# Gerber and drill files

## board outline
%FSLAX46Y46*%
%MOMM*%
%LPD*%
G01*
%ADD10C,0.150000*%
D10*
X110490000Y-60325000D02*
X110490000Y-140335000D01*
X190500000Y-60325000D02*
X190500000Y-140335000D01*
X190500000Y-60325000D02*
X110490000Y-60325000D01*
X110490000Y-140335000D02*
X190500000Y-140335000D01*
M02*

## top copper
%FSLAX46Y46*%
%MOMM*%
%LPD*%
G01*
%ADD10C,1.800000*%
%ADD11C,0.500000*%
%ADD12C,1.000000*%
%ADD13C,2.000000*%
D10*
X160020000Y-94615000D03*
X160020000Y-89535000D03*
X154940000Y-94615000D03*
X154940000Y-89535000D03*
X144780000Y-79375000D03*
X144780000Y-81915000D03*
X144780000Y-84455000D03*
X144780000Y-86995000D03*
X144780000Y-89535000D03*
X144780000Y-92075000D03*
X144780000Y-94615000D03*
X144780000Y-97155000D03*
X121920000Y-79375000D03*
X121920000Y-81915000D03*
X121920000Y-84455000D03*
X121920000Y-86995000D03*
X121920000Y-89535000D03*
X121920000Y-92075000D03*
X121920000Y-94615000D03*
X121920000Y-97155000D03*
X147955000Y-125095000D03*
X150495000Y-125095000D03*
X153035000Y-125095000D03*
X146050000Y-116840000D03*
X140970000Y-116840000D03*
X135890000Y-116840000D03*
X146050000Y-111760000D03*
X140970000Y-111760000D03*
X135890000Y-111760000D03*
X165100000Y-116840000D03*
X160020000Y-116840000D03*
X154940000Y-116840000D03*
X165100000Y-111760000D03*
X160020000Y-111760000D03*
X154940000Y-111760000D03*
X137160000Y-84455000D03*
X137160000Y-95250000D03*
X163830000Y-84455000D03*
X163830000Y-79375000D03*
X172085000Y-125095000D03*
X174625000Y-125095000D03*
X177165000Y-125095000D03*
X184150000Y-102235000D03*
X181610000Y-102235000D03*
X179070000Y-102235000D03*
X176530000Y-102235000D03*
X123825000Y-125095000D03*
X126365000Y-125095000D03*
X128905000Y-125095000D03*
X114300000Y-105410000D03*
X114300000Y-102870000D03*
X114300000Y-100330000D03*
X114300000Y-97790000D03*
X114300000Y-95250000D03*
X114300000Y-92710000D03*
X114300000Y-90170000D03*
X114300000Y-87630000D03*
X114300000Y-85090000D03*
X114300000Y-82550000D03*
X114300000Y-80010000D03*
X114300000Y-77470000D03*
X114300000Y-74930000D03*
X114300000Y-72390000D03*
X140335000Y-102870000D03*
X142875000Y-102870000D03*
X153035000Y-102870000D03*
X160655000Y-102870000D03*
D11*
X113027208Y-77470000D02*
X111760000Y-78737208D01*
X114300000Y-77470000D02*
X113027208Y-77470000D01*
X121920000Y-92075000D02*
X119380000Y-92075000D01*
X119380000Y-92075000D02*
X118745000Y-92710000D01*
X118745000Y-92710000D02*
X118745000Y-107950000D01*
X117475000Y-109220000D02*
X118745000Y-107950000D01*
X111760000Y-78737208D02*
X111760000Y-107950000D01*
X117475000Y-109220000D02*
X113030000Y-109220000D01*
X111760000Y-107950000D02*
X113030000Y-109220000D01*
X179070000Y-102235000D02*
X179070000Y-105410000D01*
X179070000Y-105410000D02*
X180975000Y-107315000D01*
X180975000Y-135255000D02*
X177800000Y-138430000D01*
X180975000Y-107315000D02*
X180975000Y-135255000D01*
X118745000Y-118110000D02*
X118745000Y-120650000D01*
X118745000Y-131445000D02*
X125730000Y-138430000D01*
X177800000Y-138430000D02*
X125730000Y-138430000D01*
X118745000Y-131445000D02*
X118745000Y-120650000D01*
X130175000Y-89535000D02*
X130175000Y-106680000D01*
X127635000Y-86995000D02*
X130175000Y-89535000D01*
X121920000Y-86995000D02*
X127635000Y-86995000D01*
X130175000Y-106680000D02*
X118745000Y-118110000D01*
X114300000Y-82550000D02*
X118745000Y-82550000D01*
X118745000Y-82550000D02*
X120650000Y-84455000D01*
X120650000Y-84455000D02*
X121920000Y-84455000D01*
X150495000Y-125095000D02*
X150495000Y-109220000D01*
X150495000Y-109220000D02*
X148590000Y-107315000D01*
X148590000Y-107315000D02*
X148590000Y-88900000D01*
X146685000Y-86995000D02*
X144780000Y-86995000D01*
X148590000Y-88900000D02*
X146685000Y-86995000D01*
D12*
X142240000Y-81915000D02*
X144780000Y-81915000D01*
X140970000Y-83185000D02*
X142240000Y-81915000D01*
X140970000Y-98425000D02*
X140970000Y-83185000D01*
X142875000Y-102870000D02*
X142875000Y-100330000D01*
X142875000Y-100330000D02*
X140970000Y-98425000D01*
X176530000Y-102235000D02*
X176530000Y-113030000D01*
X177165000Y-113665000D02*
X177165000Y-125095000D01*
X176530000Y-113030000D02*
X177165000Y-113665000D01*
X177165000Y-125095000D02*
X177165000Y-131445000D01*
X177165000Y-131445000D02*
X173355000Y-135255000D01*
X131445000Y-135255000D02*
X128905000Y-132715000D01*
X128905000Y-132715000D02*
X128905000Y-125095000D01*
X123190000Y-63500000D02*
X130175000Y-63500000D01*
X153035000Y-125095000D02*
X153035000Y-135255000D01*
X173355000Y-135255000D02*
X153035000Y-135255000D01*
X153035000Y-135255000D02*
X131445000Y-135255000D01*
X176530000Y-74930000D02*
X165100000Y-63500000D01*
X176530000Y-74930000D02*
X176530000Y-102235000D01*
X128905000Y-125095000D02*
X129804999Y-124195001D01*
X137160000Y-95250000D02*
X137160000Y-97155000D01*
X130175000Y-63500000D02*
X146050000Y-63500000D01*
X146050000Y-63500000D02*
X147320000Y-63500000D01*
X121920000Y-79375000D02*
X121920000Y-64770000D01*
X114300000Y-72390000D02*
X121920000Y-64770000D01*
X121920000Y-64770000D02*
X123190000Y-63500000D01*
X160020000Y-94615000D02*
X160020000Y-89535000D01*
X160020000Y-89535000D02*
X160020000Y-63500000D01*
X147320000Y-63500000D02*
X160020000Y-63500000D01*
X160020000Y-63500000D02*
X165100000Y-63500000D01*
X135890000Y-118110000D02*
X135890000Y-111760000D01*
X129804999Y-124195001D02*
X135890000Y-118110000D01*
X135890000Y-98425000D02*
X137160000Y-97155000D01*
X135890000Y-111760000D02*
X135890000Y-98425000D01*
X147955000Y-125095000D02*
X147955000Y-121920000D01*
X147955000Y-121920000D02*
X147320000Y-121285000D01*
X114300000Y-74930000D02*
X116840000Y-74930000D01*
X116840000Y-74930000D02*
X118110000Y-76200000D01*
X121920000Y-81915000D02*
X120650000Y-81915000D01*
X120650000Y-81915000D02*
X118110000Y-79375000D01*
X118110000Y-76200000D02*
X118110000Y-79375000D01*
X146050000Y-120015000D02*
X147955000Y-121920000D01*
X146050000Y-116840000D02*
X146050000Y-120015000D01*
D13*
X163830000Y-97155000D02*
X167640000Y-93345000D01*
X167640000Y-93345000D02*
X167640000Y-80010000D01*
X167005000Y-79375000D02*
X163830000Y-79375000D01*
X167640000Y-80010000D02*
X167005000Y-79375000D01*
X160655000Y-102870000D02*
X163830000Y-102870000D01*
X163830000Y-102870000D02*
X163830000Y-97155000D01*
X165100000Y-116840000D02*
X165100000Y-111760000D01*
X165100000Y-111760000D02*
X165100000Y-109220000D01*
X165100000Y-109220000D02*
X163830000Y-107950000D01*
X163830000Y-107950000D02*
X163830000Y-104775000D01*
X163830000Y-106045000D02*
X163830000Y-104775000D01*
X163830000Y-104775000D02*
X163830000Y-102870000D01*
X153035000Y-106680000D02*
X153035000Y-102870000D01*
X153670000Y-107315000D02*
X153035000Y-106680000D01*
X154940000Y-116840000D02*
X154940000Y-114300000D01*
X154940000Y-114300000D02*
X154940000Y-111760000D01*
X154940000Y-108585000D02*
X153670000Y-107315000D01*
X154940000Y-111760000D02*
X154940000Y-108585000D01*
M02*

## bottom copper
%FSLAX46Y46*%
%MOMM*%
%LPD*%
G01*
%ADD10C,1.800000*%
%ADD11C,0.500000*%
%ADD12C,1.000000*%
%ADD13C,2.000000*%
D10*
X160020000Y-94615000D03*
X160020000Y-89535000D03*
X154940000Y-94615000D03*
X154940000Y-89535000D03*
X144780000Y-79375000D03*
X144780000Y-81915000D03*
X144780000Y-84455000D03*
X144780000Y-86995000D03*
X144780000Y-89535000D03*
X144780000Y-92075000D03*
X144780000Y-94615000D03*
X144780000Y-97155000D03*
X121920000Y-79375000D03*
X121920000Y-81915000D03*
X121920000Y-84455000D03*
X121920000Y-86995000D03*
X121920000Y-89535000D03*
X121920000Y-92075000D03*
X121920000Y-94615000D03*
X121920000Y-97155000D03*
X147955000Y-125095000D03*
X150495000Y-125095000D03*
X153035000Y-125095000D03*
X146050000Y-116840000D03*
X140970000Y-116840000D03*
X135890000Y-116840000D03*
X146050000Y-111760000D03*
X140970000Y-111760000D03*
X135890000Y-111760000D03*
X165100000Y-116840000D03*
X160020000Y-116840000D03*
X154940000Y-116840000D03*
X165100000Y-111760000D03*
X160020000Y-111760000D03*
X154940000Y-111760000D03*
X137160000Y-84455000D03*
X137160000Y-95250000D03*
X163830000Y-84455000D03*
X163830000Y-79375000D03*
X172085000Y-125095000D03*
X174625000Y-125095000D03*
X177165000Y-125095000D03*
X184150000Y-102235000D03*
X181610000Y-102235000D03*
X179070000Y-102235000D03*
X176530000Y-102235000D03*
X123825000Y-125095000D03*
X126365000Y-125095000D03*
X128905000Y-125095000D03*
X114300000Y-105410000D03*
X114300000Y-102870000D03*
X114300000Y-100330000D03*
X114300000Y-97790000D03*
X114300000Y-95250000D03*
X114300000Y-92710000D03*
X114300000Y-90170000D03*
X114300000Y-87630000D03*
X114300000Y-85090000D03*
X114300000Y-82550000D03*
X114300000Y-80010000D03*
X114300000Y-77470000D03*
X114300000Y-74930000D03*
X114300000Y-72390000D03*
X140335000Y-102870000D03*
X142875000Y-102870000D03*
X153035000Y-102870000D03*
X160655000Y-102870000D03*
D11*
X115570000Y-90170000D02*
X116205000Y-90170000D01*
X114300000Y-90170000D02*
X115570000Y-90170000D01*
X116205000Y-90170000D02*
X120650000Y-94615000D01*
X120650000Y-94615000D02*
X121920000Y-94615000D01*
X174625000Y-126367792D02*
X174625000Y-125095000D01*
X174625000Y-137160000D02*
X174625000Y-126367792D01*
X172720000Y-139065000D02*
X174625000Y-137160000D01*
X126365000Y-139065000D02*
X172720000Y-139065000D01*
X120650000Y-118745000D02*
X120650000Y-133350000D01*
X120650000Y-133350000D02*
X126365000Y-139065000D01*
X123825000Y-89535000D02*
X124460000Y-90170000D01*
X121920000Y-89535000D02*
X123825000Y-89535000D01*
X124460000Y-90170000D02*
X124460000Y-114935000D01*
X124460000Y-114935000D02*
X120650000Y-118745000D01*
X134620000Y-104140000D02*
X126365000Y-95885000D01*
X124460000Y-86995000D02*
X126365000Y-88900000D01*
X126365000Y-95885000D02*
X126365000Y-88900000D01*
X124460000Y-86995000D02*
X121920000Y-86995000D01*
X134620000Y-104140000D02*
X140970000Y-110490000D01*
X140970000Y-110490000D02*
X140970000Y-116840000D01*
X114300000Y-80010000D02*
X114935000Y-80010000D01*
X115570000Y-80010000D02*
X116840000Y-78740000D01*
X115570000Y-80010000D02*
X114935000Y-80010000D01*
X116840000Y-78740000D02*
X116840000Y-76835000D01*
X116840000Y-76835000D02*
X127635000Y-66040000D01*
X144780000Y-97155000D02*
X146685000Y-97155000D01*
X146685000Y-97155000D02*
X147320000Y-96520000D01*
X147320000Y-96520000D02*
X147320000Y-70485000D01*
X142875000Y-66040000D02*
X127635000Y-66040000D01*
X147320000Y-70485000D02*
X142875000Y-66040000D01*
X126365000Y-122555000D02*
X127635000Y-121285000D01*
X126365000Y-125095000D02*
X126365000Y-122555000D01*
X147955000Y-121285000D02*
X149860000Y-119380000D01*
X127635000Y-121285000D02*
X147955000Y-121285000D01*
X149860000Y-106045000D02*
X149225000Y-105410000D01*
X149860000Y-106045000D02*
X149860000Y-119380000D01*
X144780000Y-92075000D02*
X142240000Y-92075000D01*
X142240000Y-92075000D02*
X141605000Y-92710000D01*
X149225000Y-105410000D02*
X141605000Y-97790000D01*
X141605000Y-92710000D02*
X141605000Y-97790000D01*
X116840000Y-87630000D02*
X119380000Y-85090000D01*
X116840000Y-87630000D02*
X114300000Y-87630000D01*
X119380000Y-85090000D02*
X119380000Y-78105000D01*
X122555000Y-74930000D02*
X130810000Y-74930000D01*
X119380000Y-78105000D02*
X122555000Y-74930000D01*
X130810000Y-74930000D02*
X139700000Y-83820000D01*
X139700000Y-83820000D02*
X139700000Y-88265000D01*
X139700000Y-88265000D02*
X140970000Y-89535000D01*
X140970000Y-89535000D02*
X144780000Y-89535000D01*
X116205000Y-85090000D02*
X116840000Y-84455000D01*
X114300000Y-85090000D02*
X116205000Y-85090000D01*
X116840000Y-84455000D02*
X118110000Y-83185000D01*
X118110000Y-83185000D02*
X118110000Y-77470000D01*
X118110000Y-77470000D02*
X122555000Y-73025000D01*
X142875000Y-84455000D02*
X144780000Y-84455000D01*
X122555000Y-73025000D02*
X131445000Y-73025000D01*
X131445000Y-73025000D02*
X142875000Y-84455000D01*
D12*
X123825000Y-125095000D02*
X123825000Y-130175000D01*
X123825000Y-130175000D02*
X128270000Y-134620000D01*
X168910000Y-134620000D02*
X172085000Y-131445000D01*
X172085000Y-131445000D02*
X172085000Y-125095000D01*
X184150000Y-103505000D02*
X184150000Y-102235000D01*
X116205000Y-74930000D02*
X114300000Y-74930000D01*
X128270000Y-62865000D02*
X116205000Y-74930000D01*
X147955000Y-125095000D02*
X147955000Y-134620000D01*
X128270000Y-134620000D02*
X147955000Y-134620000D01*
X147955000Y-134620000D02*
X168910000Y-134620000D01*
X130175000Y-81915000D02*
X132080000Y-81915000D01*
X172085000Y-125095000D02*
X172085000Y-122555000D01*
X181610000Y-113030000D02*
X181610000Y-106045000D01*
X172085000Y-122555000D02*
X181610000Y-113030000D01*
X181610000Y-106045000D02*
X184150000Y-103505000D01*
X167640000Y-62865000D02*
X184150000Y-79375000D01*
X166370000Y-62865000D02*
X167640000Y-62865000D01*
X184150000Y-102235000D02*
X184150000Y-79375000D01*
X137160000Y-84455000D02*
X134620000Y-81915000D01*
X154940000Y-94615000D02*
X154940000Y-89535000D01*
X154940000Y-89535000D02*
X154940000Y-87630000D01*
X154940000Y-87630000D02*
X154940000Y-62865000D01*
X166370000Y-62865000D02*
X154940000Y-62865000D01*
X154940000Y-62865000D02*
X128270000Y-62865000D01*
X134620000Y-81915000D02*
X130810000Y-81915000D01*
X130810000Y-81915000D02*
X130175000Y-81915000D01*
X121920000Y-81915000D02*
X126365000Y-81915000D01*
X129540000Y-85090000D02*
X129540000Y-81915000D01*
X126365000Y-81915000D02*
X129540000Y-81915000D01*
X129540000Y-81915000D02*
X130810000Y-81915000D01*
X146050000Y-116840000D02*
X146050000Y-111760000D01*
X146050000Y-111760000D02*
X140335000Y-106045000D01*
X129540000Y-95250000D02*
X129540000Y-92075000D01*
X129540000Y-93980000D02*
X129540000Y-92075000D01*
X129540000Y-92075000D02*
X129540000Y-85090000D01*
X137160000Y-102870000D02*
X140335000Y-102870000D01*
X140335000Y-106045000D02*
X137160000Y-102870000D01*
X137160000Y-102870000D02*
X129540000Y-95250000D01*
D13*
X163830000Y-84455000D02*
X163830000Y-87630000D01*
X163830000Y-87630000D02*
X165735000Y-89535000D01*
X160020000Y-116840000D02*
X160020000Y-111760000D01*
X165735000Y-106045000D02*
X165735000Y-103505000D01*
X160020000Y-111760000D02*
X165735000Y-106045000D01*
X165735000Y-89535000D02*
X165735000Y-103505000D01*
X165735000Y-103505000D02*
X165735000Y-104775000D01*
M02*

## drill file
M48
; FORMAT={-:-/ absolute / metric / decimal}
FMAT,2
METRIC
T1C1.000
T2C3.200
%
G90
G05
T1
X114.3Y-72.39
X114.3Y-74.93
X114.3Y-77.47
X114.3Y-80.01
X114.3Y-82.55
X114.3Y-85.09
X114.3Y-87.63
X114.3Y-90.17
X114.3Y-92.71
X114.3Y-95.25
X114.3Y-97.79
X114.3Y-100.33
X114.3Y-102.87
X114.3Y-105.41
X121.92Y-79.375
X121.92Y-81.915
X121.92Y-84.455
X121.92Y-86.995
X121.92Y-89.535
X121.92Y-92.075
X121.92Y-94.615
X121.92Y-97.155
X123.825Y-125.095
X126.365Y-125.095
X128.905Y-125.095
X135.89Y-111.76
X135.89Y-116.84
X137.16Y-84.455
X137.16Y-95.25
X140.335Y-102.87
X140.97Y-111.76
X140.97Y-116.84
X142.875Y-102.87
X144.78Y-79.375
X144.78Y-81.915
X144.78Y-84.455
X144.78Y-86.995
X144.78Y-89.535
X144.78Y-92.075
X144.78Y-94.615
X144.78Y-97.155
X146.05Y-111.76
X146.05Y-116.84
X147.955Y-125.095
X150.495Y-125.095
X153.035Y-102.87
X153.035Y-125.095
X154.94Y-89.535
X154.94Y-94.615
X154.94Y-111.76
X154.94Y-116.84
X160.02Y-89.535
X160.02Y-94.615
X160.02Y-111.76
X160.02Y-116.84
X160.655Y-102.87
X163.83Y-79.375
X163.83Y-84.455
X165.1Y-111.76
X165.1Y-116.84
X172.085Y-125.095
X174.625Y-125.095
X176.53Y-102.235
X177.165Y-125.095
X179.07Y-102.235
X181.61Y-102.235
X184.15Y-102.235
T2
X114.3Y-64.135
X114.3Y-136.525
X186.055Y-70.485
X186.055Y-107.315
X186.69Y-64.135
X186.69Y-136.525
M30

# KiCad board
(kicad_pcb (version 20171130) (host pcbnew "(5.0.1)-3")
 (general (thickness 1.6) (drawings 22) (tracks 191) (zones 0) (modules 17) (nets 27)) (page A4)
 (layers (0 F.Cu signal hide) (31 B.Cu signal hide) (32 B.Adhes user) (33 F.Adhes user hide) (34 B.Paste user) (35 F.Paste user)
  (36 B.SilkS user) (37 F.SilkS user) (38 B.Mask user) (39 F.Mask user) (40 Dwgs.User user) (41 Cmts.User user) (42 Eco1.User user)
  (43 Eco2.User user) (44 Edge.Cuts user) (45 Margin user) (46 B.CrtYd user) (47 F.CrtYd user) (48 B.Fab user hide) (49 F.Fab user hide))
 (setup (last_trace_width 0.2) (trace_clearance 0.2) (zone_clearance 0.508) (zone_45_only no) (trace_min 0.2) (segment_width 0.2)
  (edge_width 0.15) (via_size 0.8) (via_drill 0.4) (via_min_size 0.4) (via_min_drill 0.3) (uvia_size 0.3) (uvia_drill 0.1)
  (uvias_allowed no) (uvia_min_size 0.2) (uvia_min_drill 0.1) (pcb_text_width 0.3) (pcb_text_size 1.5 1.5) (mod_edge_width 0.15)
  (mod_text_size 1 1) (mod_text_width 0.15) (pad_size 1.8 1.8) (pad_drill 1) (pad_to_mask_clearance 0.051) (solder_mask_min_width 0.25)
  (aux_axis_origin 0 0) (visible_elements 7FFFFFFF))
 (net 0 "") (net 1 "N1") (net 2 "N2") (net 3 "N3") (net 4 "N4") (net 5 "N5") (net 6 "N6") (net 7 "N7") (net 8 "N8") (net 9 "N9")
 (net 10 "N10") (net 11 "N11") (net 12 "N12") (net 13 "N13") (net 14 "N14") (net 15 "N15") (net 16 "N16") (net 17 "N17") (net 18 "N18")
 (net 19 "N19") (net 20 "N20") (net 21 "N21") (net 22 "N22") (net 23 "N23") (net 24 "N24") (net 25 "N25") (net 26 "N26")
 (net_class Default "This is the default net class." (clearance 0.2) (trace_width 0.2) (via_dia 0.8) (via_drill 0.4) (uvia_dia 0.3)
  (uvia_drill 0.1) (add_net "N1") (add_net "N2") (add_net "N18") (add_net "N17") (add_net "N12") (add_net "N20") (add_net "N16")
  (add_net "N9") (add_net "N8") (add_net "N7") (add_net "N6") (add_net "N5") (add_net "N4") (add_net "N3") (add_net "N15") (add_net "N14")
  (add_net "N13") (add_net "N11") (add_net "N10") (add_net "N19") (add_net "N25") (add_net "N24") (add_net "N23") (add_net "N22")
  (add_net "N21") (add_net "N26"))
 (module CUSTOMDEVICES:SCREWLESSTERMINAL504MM (layer B.Cu) (at 154.94 92.075 180)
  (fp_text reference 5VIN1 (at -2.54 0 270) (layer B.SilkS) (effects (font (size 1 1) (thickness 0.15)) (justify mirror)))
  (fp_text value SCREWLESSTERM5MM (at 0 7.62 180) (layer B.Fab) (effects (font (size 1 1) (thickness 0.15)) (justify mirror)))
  (pad 1 thru_hole circle (at -5.08 -2.54 180) (size 1.8 1.8) (drill 1) (layers *.Cu *.Mask) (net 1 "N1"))
  (pad 1 thru_hole circle (at -5.08 2.54 180) (size 1.8 1.8) (drill 1) (layers *.Cu *.Mask) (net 1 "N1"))
  (pad 2 thru_hole circle (at 0 -2.54 180) (size 1.8 1.8) (drill 1) (layers *.Cu *.Mask) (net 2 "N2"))
  (pad 2 thru_hole circle (at 0 2.54 180) (size 1.8 1.8) (drill 1) (layers *.Cu *.Mask) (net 2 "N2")))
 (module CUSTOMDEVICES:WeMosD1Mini (layer F.Cu) (at 133.35 86.995 180)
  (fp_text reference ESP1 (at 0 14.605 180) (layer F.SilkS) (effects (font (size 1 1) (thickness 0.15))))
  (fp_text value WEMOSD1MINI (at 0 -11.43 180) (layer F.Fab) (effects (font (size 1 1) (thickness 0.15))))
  (pad 16 thru_hole circle (at -11.43 7.62 180) (size 1.8 1.8) (drill 1) (layers *.Cu *.Mask) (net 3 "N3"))
  (pad 15 thru_hole circle (at -11.43 5.08 180) (size 1.8 1.8) (drill 1) (layers *.Cu *.Mask) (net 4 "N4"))
  (pad 14 thru_hole circle (at -11.43 2.54 180) (size 1.8 1.8) (drill 1) (layers *.Cu *.Mask) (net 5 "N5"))
  (pad 13 thru_hole circle (at -11.43 0 180) (size 1.8 1.8) (drill 1) (layers *.Cu *.Mask) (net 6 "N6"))
  (pad 12 thru_hole circle (at -11.43 -2.54 180) (size 1.8 1.8) (drill 1) (layers *.Cu *.Mask) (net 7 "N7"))
  (pad 11 thru_hole circle (at -11.43 -5.08 180) (size 1.8 1.8) (drill 1) (layers *.Cu *.Mask) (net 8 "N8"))
  (pad 10 thru_hole circle (at -11.43 -7.62 180) (size 1.8 1.8) (drill 1) (layers *.Cu *.Mask) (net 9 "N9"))
  (pad 9 thru_hole circle (at -11.43 -10.16 180) (size 1.8 1.8) (drill 1) (layers *.Cu *.Mask) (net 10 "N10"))
  (pad 8 thru_hole circle (at 11.43 7.62 180) (size 1.8 1.8) (drill 1) (layers *.Cu *.Mask) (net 1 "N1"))
  (pad 7 thru_hole circle (at 11.43 5.08 180) (size 1.8 1.8) (drill 1) (layers *.Cu *.Mask) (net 2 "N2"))
  (pad 6 thru_hole circle (at 11.43 2.54 180) (size 1.8 1.8) (drill 1) (layers *.Cu *.Mask) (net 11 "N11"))
  (pad 5 thru_hole circle (at 11.43 0 180) (size 1.8 1.8) (drill 1) (layers *.Cu *.Mask) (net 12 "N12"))
  (pad 4 thru_hole circle (at 11.43 -2.54 180) (size 1.8 1.8) (drill 1) (layers *.Cu *.Mask) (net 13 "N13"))
  (pad 3 thru_hole circle (at 11.43 -5.08 180) (size 1.8 1.8) (drill 1) (layers *.Cu *.Mask) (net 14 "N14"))
  (pad 2 thru_hole circle (at 11.43 -7.62 180) (size 1.8 1.8) (drill 1) (layers *.Cu *.Mask) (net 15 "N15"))
  (pad 1 thru_hole circle (at 11.43 -10.16 180) (size 1.8 1.8) (drill 1) (layers *.Cu *.Mask) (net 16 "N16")))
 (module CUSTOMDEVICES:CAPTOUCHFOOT (layer F.Cu) (at 150.495 130.175 180)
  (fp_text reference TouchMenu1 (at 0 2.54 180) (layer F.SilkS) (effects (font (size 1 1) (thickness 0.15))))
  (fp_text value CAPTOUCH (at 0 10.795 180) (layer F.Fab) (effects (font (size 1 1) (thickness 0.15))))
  (pad 3 thru_hole circle (at 2.54 5.08 180) (size 1.8 1.8) (drill 1) (layers *.Cu *.Mask) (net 2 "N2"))
  (pad 2 thru_hole circle (at 0 5.08 180) (size 1.8 1.8) (drill 1) (layers *.Cu *.Mask) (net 6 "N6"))
  (pad 1 thru_hole circle (at -2.54 5.08 180) (size 1.8 1.8) (drill 1) (layers *.Cu *.Mask) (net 1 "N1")))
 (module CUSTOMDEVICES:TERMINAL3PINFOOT (layer B.Cu) (at 140.97 114.3)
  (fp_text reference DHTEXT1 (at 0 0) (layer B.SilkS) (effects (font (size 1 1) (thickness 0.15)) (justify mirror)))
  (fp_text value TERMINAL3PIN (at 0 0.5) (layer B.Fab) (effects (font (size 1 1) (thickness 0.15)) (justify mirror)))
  (pad 3 thru_hole circle (at 5.08 2.54) (size 1.8 1.8) (drill 1) (layers *.Cu *.Mask) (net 2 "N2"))
  (pad 2 thru_hole circle (at 0 2.54) (size 1.8 1.8) (drill 1) (layers *.Cu *.Mask) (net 12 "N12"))
  (pad 1 thru_hole circle (at -5.08 2.54) (size 1.8 1.8) (drill 1) (layers *.Cu *.Mask) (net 1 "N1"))
  (pad 3 thru_hole circle (at 5.08 -2.54) (size 1.8 1.8) (drill 1) (layers *.Cu *.Mask) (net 2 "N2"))
  (pad 2 thru_hole circle (at 0 -2.54) (size 1.8 1.8) (drill 1) (layers *.Cu *.Mask) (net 12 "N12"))
  (pad 1 thru_hole circle (at -5.08 -2.54) (size 1.8 1.8) (drill 1) (layers *.Cu *.Mask) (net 1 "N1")))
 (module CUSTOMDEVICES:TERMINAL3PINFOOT (layer B.Cu) (at 160.02 114.3)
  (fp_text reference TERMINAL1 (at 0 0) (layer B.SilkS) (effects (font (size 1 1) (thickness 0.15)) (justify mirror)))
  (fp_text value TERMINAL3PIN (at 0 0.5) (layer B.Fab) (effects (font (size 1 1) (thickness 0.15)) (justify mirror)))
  (pad 3 thru_hole circle (at 5.08 2.54) (size 1.8 1.8) (drill 1) (layers *.Cu *.Mask) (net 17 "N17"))
  (pad 2 thru_hole circle (at 0 2.54) (size 1.8 1.8) (drill 1) (layers *.Cu *.Mask) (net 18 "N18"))
  (pad 1 thru_hole circle (at -5.08 2.54) (size 1.8 1.8) (drill 1) (layers *.Cu *.Mask) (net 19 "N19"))
  (pad 3 thru_hole circle (at 5.08 -2.54) (size 1.8 1.8) (drill 1) (layers *.Cu *.Mask) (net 17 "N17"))
  (pad 2 thru_hole circle (at 0 -2.54) (size 1.8 1.8) (drill 1) (layers *.Cu *.Mask) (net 18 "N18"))
  (pad 1 thru_hole circle (at -5.08 -2.54) (size 1.8 1.8) (drill 1) (layers *.Cu *.Mask) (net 19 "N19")))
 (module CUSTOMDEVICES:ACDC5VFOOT (layer B.Cu) (at 157.48 86.995 90)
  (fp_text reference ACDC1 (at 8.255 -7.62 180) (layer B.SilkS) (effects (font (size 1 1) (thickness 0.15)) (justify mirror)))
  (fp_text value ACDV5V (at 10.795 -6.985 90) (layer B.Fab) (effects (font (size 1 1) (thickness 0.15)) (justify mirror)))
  (pad 3 thru_hole circle (at 2.54 -20.32 90) (size 1.8 1.8) (drill 1) (layers *.Cu *.Mask) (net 2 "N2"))
  (pad 4 thru_hole circle (at -8.255 -20.32 90) (size 1.8 1.8) (drill 1) (layers *.Cu *.Mask) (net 1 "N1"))
  (pad 1 thru_hole circle (at 2.54 6.35 90) (size 1.8 1.8) (drill 1) (layers *.Cu *.Mask) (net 18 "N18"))
  (pad 2 thru_hole circle (at 7.62 6.35 90) (size 1.8 1.8) (drill 1) (layers *.Cu *.Mask) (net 17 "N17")))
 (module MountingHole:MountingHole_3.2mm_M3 (layer F.Cu) (at 186.055 107.315)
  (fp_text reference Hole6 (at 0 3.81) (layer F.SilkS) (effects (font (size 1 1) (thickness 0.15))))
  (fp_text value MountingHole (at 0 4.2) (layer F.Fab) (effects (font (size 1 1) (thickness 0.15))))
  (pad 1 np_thru_hole circle (at 0 0) (size 3.2 3.2) (drill 3.2) (layers *.Cu *.Mask)))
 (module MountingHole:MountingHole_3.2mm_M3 (layer F.Cu) (at 186.055 70.485)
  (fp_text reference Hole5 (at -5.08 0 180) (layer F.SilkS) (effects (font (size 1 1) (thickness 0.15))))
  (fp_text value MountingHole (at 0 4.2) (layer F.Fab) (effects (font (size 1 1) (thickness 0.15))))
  (pad 1 np_thru_hole circle (at 0 0) (size 3.2 3.2) (drill 3.2) (layers *.Cu *.Mask)))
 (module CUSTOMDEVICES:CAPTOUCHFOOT (layer F.Cu) (at 174.625 130.175 180)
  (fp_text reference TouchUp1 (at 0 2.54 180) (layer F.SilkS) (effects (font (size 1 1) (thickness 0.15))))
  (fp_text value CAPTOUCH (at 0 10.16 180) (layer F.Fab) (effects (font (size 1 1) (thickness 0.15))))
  (pad 3 thru_hole circle (at 2.54 5.08 180) (size 1.8 1.8) (drill 1) (layers *.Cu *.Mask) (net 2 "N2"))
  (pad 2 thru_hole circle (at 0 5.08 180) (size 1.8 1.8) (drill 1) (layers *.Cu *.Mask) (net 13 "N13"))
  (pad 1 thru_hole circle (at -2.54 5.08 180) (size 1.8 1.8) (drill 1) (layers *.Cu *.Mask) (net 1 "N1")))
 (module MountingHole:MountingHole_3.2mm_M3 (layer F.Cu) (at 186.69 136.525)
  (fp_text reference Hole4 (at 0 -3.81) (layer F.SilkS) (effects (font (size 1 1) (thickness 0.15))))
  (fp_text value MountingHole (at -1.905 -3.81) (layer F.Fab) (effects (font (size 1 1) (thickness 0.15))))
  (pad 1 np_thru_hole circle (at 0 0) (size 3.2 3.2) (drill 3.2) (layers *.Cu *.Mask)))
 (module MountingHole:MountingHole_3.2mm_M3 (layer F.Cu) (at 114.3 136.525)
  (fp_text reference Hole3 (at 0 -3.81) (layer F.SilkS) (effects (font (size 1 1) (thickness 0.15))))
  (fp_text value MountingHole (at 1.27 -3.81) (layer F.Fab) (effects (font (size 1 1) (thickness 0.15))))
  (pad 1 np_thru_hole circle (at 0 0) (size 3.2 3.2) (drill 3.2) (layers *.Cu *.Mask)))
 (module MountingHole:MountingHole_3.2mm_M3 (layer F.Cu) (at 186.69 64.135)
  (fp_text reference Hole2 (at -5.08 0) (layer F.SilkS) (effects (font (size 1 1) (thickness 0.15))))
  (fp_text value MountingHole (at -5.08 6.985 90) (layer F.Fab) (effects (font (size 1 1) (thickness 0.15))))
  (pad 1 np_thru_hole circle (at 0 0) (size 3.2 3.2) (drill 3.2) (layers *.Cu *.Mask)))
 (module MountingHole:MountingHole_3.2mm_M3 (layer F.Cu) (at 114.3 64.135)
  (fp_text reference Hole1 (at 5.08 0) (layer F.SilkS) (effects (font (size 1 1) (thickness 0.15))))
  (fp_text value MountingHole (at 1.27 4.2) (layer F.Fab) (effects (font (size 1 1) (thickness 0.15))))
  (pad 1 np_thru_hole circle (at 0 0) (size 3.2 3.2) (drill 3.2) (layers *.Cu *.Mask)))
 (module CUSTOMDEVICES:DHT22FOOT (layer F.Cu) (at 181.61 89.535)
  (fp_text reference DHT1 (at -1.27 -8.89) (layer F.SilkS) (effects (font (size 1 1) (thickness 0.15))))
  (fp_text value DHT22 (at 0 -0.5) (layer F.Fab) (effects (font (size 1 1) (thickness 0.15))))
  (pad 4 thru_hole circle (at 2.54 12.7) (size 1.8 1.8) (drill 1) (layers *.Cu *.Mask) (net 2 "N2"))
  (pad 3 thru_hole circle (at 0 12.7) (size 1.8 1.8) (drill 1) (layers *.Cu *.Mask) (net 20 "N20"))
  (pad 2 thru_hole circle (at -2.54 12.7) (size 1.8 1.8) (drill 1) (layers *.Cu *.Mask) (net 12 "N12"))
  (pad 1 thru_hole circle (at -5.08 12.7) (size 1.8 1.8) (drill 1) (layers *.Cu *.Mask) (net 1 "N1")))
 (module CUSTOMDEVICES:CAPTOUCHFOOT (layer F.Cu) (at 126.365 130.175 180)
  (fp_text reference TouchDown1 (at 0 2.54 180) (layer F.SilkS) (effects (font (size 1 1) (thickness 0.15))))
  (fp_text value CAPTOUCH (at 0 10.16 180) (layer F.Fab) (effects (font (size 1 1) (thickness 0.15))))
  (pad 3 thru_hole circle (at 2.54 5.08 180) (size 1.8 1.8) (drill 1) (layers *.Cu *.Mask) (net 2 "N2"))
  (pad 2 thru_hole circle (at 0 5.08 180) (size 1.8 1.8) (drill 1) (layers *.Cu *.Mask) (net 8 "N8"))
  (pad 1 thru_hole circle (at -2.54 5.08 180) (size 1.8 1.8) (drill 1) (layers *.Cu *.Mask) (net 1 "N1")))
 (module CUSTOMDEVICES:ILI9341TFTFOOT (layer F.Cu) (at 116.84 90.17 180)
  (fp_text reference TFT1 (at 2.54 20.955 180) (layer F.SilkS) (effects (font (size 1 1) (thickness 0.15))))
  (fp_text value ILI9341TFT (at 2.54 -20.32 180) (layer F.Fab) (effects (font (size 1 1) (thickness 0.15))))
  (pad 14 thru_hole circle (at 2.54 -15.24 180) (size 1.8 1.8) (drill 1) (layers *.Cu *.Mask) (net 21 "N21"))
  (pad 13 thru_hole circle (at 2.54 -12.7 180) (size 1.8 1.8) (drill 1) (layers *.Cu *.Mask) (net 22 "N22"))
  (pad 12 thru_hole circle (at 2.54 -10.16 180) (size 1.8 1.8) (drill 1) (layers *.Cu *.Mask) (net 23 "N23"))
  (pad 11 thru_hole circle (at 2.54 -7.62 180) (size 1.8 1.8) (drill 1) (layers *.Cu *.Mask) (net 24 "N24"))
  (pad 10 thru_hole circle (at 2.54 -5.08 180) (size 1.8 1.8) (drill 1) (layers *.Cu *.Mask) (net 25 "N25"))
  (pad 9 thru_hole circle (at 2.54 -2.54 180) (size 1.8 1.8) (drill 1) (layers *.Cu *.Mask) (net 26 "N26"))
  (pad 8 thru_hole circle (at 2.54 0 180) (size 1.8 1.8) (drill 1) (layers *.Cu *.Mask) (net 15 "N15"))
  (pad 7 thru_hole circle (at 2.54 2.54 180) (size 1.8 1.8) (drill 1) (layers *.Cu *.Mask) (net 7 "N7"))
  (pad 6 thru_hole circle (at 2.54 5.08 180) (size 1.8 1.8) (drill 1) (layers *.Cu *.Mask) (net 5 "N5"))
  (pad 5 thru_hole circle (at 2.54 7.62 180) (size 1.8 1.8) (drill 1) (layers *.Cu *.Mask) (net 11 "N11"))
  (pad 4 thru_hole circle (at 2.54 10.16 180) (size 1.8 1.8) (drill 1) (layers *.Cu *.Mask) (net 10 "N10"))
  (pad 3 thru_hole circle (at 2.54 12.7 180) (size 1.8 1.8) (drill 1) (layers *.Cu *.Mask) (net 14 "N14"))
  (pad 2 thru_hole circle (at 2.54 15.24 180) (size 1.8 1.8) (drill 1) (layers *.Cu *.Mask) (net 2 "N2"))
  (pad 1 thru_hole circle (at 2.54 17.78 180) (size 1.8 1.8) (drill 1) (layers *.Cu *.Mask) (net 1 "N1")))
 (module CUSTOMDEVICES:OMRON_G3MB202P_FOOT (layer B.Cu) (at 150.495 102.87 90)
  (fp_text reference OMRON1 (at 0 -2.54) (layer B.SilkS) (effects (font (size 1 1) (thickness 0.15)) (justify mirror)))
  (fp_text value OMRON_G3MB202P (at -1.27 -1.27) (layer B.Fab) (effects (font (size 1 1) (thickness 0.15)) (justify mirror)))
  (pad 4 thru_hole circle (at 0 -10.16 90) (size 1.8 1.8) (drill 1) (layers *.Cu *.Mask) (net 2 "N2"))
  (pad 3 thru_hole circle (at 0 -7.62 90) (size 1.8 1.8) (drill 1) (layers *.Cu *.Mask) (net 4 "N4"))
  (pad 2 thru_hole circle (at 0 2.54 90) (size 1.8 1.8) (drill 1) (layers *.Cu *.Mask) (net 19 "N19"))
  (pad 1 thru_hole circle (at 0 10.16 90) (size 1.8 1.8) (drill 1) (layers *.Cu *.Mask) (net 17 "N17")))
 (gr_line (start 110.49 60.325) (end 110.49 140.335) (layer Edge.Cuts) (width 0.15))
 (gr_line (start 190.5 60.325) (end 190.5 140.335) (layer Edge.Cuts) (width 0.15))
 (gr_line (start 190.5 60.325) (end 110.49 60.325) (layer Edge.Cuts) (width 0.15))
 (gr_line (start 110.49 140.335) (end 190.5 140.335) (layer Edge.Cuts) (width 0.15))
 (segment (start 115.57 90.17) (end 116.205 90.17) (width 0.5) (layer B.Cu) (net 15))
 (segment (start 114.3 90.17) (end 115.57 90.17) (width 0.5) (layer B.Cu) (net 15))
 (segment (start 116.205 90.17) (end 120.65 94.615) (width 0.5) (layer B.Cu) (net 15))
 (segment (start 120.65 94.615) (end 121.92 94.615) (width 0.5) (layer B.Cu) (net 15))
 (segment (start 113.027208 77.47) (end 111.76 78.737208) (width 0.5) (layer F.Cu) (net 14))
 (segment (start 114.3 77.47) (end 113.027208 77.47) (width 0.5) (layer F.Cu) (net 14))
 (segment (start 121.92 92.075) (end 119.38 92.075) (width 0.5) (layer F.Cu) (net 14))
 (segment (start 119.38 92.075) (end 118.745 92.71) (width 0.5) (layer F.Cu) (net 14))
 (segment (start 118.745 92.71) (end 118.745 107.95) (width 0.5) (layer F.Cu) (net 14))
 (segment (start 117.475 109.22) (end 118.745 107.95) (width 0.5) (layer F.Cu) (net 14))
 (segment (start 111.76 78.737208) (end 111.76 107.95) (width 0.5) (layer F.Cu) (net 14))
 (segment (start 117.475 109.22) (end 113.03 109.22) (width 0.5) (layer F.Cu) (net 14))
 (segment (start 111.76 107.95) (end 113.03 109.22) (width 0.5) (layer F.Cu) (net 14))
 (segment (start 174.625 126.367792) (end 174.625 125.095) (width 0.5) (layer B.Cu) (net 13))
 (segment (start 174.625 137.16) (end 174.625 126.367792) (width 0.5) (layer B.Cu) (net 13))
 (segment (start 172.72 139.065) (end 174.625 137.16) (width 0.5) (layer B.Cu) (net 13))
 (segment (start 126.365 139.065) (end 172.72 139.065) (width 0.5) (layer B.Cu) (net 13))
 (segment (start 120.65 118.745) (end 120.65 133.35) (width 0.5) (layer B.Cu) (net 13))
 (segment (start 120.65 133.35) (end 126.365 139.065) (width 0.5) (layer B.Cu) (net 13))
 (segment (start 123.825 89.535) (end 124.46 90.17) (width 0.5) (layer B.Cu) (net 13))
 (segment (start 121.92 89.535) (end 123.825 89.535) (width 0.5) (layer B.Cu) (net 13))
 (segment (start 124.46 90.17) (end 124.46 114.935) (width 0.5) (layer B.Cu) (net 13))
 (segment (start 124.46 114.935) (end 120.65 118.745) (width 0.5) (layer B.Cu) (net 13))
 (segment (start 179.07 102.235) (end 179.07 105.41) (width 0.5) (layer F.Cu) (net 12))
 (segment (start 179.07 105.41) (end 180.975 107.315) (width 0.5) (layer F.Cu) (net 12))
 (segment (start 180.975 135.255) (end 177.8 138.43) (width 0.5) (layer F.Cu) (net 12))
 (segment (start 180.975 107.315) (end 180.975 135.255) (width 0.5) (layer F.Cu) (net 12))
 (segment (start 118.745 118.11) (end 118.745 120.65) (width 0.5) (layer F.Cu) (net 12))
 (segment (start 118.745 131.445) (end 125.73 138.43) (width 0.5) (layer F.Cu) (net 12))
 (segment (start 177.8 138.43) (end 125.73 138.43) (width 0.5) (layer F.Cu) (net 12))
 (segment (start 118.745 131.445) (end 118.745 120.65) (width 0.5) (layer F.Cu) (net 12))
 (segment (start 130.175 89.535) (end 130.175 106.68) (width 0.5) (layer F.Cu) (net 12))
 (segment (start 127.635 86.995) (end 130.175 89.535) (width 0.5) (layer F.Cu) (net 12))
 (segment (start 121.92 86.995) (end 127.635 86.995) (width 0.5) (layer F.Cu) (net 12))
 (segment (start 130.175 106.68) (end 118.745 118.11) (width 0.5) (layer F.Cu) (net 12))
 (segment (start 134.62 104.14) (end 126.365 95.885) (width 0.5) (layer B.Cu) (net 12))
 (segment (start 124.46 86.995) (end 126.365 88.9) (width 0.5) (layer B.Cu) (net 12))
 (segment (start 126.365 95.885) (end 126.365 88.9) (width 0.5) (layer B.Cu) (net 12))
 (segment (start 124.46 86.995) (end 121.92 86.995) (width 0.5) (layer B.Cu) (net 12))
 (segment (start 134.62 104.14) (end 140.97 110.49) (width 0.5) (layer B.Cu) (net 12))
 (segment (start 140.97 110.49) (end 140.97 116.84) (width 0.5) (layer B.Cu) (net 12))
 (segment (start 114.3 82.55) (end 118.745 82.55) (width 0.5) (layer F.Cu) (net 11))
 (segment (start 118.745 82.55) (end 120.65 84.455) (width 0.5) (layer F.Cu) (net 11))
 (segment (start 120.65 84.455) (end 121.92 84.455) (width 0.5) (layer F.Cu) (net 11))
 (segment (start 114.3 80.01) (end 114.935 80.01) (width 0.5) (layer B.Cu) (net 10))
 (segment (start 115.57 80.01) (end 116.84 78.74) (width 0.5) (layer B.Cu) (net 10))
 (segment (start 115.57 80.01) (end 114.935 80.01) (width 0.5) (layer B.Cu) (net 10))
 (segment (start 116.84 78.74) (end 116.84 76.835) (width 0.5) (layer B.Cu) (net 10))
 (segment (start 116.84 76.835) (end 127.635 66.04) (width 0.5) (layer B.Cu) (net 10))
 (segment (start 144.78 97.155) (end 146.685 97.155) (width 0.5) (layer B.Cu) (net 10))
 (segment (start 146.685 97.155) (end 147.32 96.52) (width 0.5) (layer B.Cu) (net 10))
 (segment (start 147.32 96.52) (end 147.32 70.485) (width 0.5) (layer B.Cu) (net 10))
 (segment (start 142.875 66.04) (end 127.635 66.04) (width 0.5) (layer B.Cu) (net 10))
 (segment (start 147.32 70.485) (end 142.875 66.04) (width 0.5) (layer B.Cu) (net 10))
 (segment (start 126.365 122.555) (end 127.635 121.285) (width 0.5) (layer B.Cu) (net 8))
 (segment (start 126.365 125.095) (end 126.365 122.555) (width 0.5) (layer B.Cu) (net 8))
 (segment (start 147.955 121.285) (end 149.86 119.38) (width 0.5) (layer B.Cu) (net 8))
 (segment (start 127.635 121.285) (end 147.955 121.285) (width 0.5) (layer B.Cu) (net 8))
 (segment (start 149.86 106.045) (end 149.225 105.41) (width 0.5) (layer B.Cu) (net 8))
 (segment (start 149.86 106.045) (end 149.86 119.38) (width 0.5) (layer B.Cu) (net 8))
 (segment (start 144.78 92.075) (end 142.24 92.075) (width 0.5) (layer B.Cu) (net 8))
 (segment (start 142.24 92.075) (end 141.605 92.71) (width 0.5) (layer B.Cu) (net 8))
 (segment (start 149.225 105.41) (end 141.605 97.79) (width 0.5) (layer B.Cu) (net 8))
 (segment (start 141.605 92.71) (end 141.605 97.79) (width 0.5) (layer B.Cu) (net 8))
 (segment (start 116.84 87.63) (end 119.38 85.09) (width 0.5) (layer B.Cu) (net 7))
 (segment (start 116.84 87.63) (end 114.3 87.63) (width 0.5) (layer B.Cu) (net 7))
 (segment (start 119.38 85.09) (end 119.38 78.105) (width 0.5) (layer B.Cu) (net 7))
 (segment (start 122.555 74.93) (end 130.81 74.93) (width 0.5) (layer B.Cu) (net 7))
 (segment (start 119.38 78.105) (end 122.555 74.93) (width 0.5) (layer B.Cu) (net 7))
 (segment (start 130.81 74.93) (end 139.7 83.82) (width 0.5) (layer B.Cu) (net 7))
 (segment (start 139.7 83.82) (end 139.7 88.265) (width 0.5) (layer B.Cu) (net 7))
 (segment (start 139.7 88.265) (end 140.97 89.535) (width 0.5) (layer B.Cu) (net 7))
 (segment (start 140.97 89.535) (end 144.78 89.535) (width 0.5) (layer B.Cu) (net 7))
 (segment (start 150.495 125.095) (end 150.495 109.22) (width 0.5) (layer F.Cu) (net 6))
 (segment (start 150.495 109.22) (end 148.59 107.315) (width 0.5) (layer F.Cu) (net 6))
 (segment (start 148.59 107.315) (end 148.59 88.9) (width 0.5) (layer F.Cu) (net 6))
 (segment (start 146.685 86.995) (end 144.78 86.995) (width 0.5) (layer F.Cu) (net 6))
 (segment (start 148.59 88.9) (end 146.685 86.995) (width 0.5) (layer F.Cu) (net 6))
 (segment (start 116.205 85.09) (end 116.84 84.455) (width 0.5) (layer B.Cu) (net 5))
 (segment (start 114.3 85.09) (end 116.205 85.09) (width 0.5) (layer B.Cu) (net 5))
 (segment (start 116.84 84.455) (end 118.11 83.185) (width 0.5) (layer B.Cu) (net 5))
 (segment (start 118.11 83.185) (end 118.11 77.47) (width 0.5) (layer B.Cu) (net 5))
 (segment (start 118.11 77.47) (end 122.555 73.025) (width 0.5) (layer B.Cu) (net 5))
 (segment (start 142.875 84.455) (end 144.78 84.455) (width 0.5) (layer B.Cu) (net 5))
 (segment (start 122.555 73.025) (end 131.445 73.025) (width 0.5) (layer B.Cu) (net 5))
 (segment (start 131.445 73.025) (end 142.875 84.455) (width 0.5) (layer B.Cu) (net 5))
 (segment (start 142.24 81.915) (end 144.78 81.915) (width 1) (layer F.Cu) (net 4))
 (segment (start 140.97 83.185) (end 142.24 81.915) (width 1) (layer F.Cu) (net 4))
 (segment (start 140.97 98.425) (end 140.97 83.185) (width 1) (layer F.Cu) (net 4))
 (segment (start 142.875 102.87) (end 142.875 100.33) (width 1) (layer F.Cu) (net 4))
 (segment (start 142.875 100.33) (end 140.97 98.425) (width 1) (layer F.Cu) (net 4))
 (segment (start 176.53 102.235) (end 176.53 113.03) (width 1) (layer F.Cu) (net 1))
 (segment (start 177.165 113.665) (end 177.165 125.095) (width 1) (layer F.Cu) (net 1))
 (segment (start 176.53 113.03) (end 177.165 113.665) (width 1) (layer F.Cu) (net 1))
 (segment (start 177.165 125.095) (end 177.165 131.445) (width 1) (layer F.Cu) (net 1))
 (segment (start 177.165 131.445) (end 173.355 135.255) (width 1) (layer F.Cu) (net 1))
 (segment (start 131.445 135.255) (end 128.905 132.715) (width 1) (layer F.Cu) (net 1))
 (segment (start 128.905 132.715) (end 128.905 125.095) (width 1) (layer F.Cu) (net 1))
 (segment (start 123.19 63.5) (end 130.175 63.5) (width 1) (layer F.Cu) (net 1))
 (segment (start 153.035 125.095) (end 153.035 135.255) (width 1) (layer F.Cu) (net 1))
 (segment (start 173.355 135.255) (end 153.035 135.255) (width 1) (layer F.Cu) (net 1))
 (segment (start 153.035 135.255) (end 131.445 135.255) (width 1) (layer F.Cu) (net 1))
 (segment (start 176.53 74.93) (end 165.1 63.5) (width 1) (layer F.Cu) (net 1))
 (segment (start 176.53 74.93) (end 176.53 102.235) (width 1) (layer F.Cu) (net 1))
 (segment (start 128.905 125.095) (end 129.804999 124.195001) (width 1) (layer F.Cu) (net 1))
 (segment (start 137.16 95.25) (end 137.16 97.155) (width 1) (layer F.Cu) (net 1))
 (segment (start 130.175 63.5) (end 146.05 63.5) (width 1) (layer F.Cu) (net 1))
 (segment (start 146.05 63.5) (end 147.32 63.5) (width 1) (layer F.Cu) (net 1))
 (segment (start 121.92 79.375) (end 121.92 64.77) (width 1) (layer F.Cu) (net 1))
 (segment (start 114.3 72.39) (end 121.92 64.77) (width 1) (layer F.Cu) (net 1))
 (segment (start 121.92 64.77) (end 123.19 63.5) (width 1) (layer F.Cu) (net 1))
 (segment (start 160.02 94.615) (end 160.02 89.535) (width 1) (layer F.Cu) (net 1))
 (segment (start 160.02 89.535) (end 160.02 63.5) (width 1) (layer F.Cu) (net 1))
 (segment (start 147.32 63.5) (end 160.02 63.5) (width 1) (layer F.Cu) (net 1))
 (segment (start 160.02 63.5) (end 165.1 63.5) (width 1) (layer F.Cu) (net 1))
 (segment (start 135.89 118.11) (end 135.89 111.76) (width 1) (layer F.Cu) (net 1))
 (segment (start 129.804999 124.195001) (end 135.89 118.11) (width 1) (layer F.Cu) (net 1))
 (segment (start 135.89 98.425) (end 137.16 97.155) (width 1) (layer F.Cu) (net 1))
 (segment (start 135.89 111.76) (end 135.89 98.425) (width 1) (layer F.Cu) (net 1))
 (segment (start 123.825 125.095) (end 123.825 130.175) (width 1) (layer B.Cu) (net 2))
 (segment (start 123.825 130.175) (end 128.27 134.62) (width 1) (layer B.Cu) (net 2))
 (segment (start 168.91 134.62) (end 172.085 131.445) (width 1) (layer B.Cu) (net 2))
 (segment (start 172.085 131.445) (end 172.085 125.095) (width 1) (layer B.Cu) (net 2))
 (segment (start 184.15 103.505) (end 184.15 102.235) (width 1) (layer B.Cu) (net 2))
 (segment (start 116.205 74.93) (end 114.3 74.93) (width 1) (layer B.Cu) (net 2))
 (segment (start 128.27 62.865) (end 116.205 74.93) (width 1) (layer B.Cu) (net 2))
 (segment (start 147.955 125.095) (end 147.955 134.62) (width 1) (layer B.Cu) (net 2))
 (segment (start 128.27 134.62) (end 147.955 134.62) (width 1) (layer B.Cu) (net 2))
 (segment (start 147.955 134.62) (end 168.91 134.62) (width 1) (layer B.Cu) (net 2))
 (segment (start 130.175 81.915) (end 132.08 81.915) (width 1) (layer B.Cu) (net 2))
 (segment (start 147.955 125.095) (end 147.955 121.92) (width 1) (layer F.Cu) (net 2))
 (segment (start 147.955 121.92) (end 147.32 121.285) (width 1) (layer F.Cu) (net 2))
 (segment (start 172.085 125.095) (end 172.085 122.555) (width 1) (layer B.Cu) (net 2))
 (segment (start 181.61 113.03) (end 181.61 106.045) (width 1) (layer B.Cu) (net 2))
 (segment (start 172.085 122.555) (end 181.61 113.03) (width 1) (layer B.Cu) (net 2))
 (segment (start 181.61 106.045) (end 184.15 103.505) (width 1) (layer B.Cu) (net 2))
 (segment (start 167.64 62.865) (end 184.15 79.375) (width 1) (layer B.Cu) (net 2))
 (segment (start 166.37 62.865) (end 167.64 62.865) (width 1) (layer B.Cu) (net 2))
 (segment (start 184.15 102.235) (end 184.15 79.375) (width 1) (layer B.Cu) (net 2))
 (segment (start 137.16 84.455) (end 134.62 81.915) (width 1) (layer B.Cu) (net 2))
 (segment (start 114.3 74.93) (end 116.84 74.93) (width 1) (layer F.Cu) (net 2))
 (segment (start 116.84 74.93) (end 118.11 76.2) (width 1) (layer F.Cu) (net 2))
 (segment (start 121.92 81.915) (end 120.65 81.915) (width 1) (layer F.Cu) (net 2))
 (segment (start 120.65 81.915) (end 118.11 79.375) (width 1) (layer F.Cu) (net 2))
 (segment (start 118.11 76.2) (end 118.11 79.375) (width 1) (layer F.Cu) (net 2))
 (segment (start 154.94 94.615) (end 154.94 89.535) (width 1) (layer B.Cu) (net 2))
 (segment (start 154.94 89.535) (end 154.94 87.63) (width 1) (layer B.Cu) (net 2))
 (segment (start 154.94 87.63) (end 154.94 62.865) (width 1) (layer B.Cu) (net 2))
 (segment (start 166.37 62.865) (end 154.94 62.865) (width 1) (layer B.Cu) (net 2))
 (segment (start 154.94 62.865) (end 128.27 62.865) (width 1) (layer B.Cu) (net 2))
 (segment (start 134.62 81.915) (end 130.81 81.915) (width 1) (layer B.Cu) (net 2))
 (segment (start 130.81 81.915) (end 130.175 81.915) (width 1) (layer B.Cu) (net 2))
 (segment (start 121.92 81.915) (end 126.365 81.915) (width 1) (layer B.Cu) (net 2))
 (segment (start 129.54 85.09) (end 129.54 81.915) (width 1) (layer B.Cu) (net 2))
 (segment (start 126.365 81.915) (end 129.54 81.915) (width 1) (layer B.Cu) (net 2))
 (segment (start 129.54 81.915) (end 130.81 81.915) (width 1) (layer B.Cu) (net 2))
 (segment (start 146.05 120.015) (end 147.955 121.92) (width 1) (layer F.Cu) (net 2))
 (segment (start 146.05 116.84) (end 146.05 120.015) (width 1) (layer F.Cu) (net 2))
 (segment (start 146.05 116.84) (end 146.05 111.76) (width 1) (layer B.Cu) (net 2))
 (segment (start 146.05 111.76) (end 140.335 106.045) (width 1) (layer B.Cu) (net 2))
 (segment (start 129.54 95.25) (end 129.54 92.075) (width 1) (layer B.Cu) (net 2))
 (segment (start 129.54 93.98) (end 129.54 92.075) (width 1) (layer B.Cu) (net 2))
 (segment (start 129.54 92.075) (end 129.54 85.09) (width 1) (layer B.Cu) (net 2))
 (segment (start 137.16 102.87) (end 140.335 102.87) (width 1) (layer B.Cu) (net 2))
 (segment (start 140.335 106.045) (end 137.16 102.87) (width 1) (layer B.Cu) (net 2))
 (segment (start 137.16 102.87) (end 129.54 95.25) (width 1) (layer B.Cu) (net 2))
 (segment (start 163.83 97.155) (end 167.64 93.345) (width 2) (layer F.Cu) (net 17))
 (segment (start 167.64 93.345) (end 167.64 80.01) (width 2) (layer F.Cu) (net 17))
 (segment (start 167.005 79.375) (end 163.83 79.375) (width 2) (layer F.Cu) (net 17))
 (segment (start 167.64 80.01) (end 167.005 79.375) (width 2) (layer F.Cu) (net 17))
 (segment (start 160.655 102.87) (end 163.83 102.87) (width 2) (layer F.Cu) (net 17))
 (segment (start 163.83 102.87) (end 163.83 97.155) (width 2) (layer F.Cu) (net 17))
 (segment (start 165.1 116.84) (end 165.1 111.76) (width 2) (layer F.Cu) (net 17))
 (segment (start 165.1 111.76) (end 165.1 109.22) (width 2) (layer F.Cu) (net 17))
 (segment (start 165.1 109.22) (end 163.83 107.95) (width 2) (layer F.Cu) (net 17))
 (segment (start 163.83 107.95) (end 163.83 104.775) (width 2) (layer F.Cu) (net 17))
 (segment (start 163.83 106.045) (end 163.83 104.775) (width 2) (layer F.Cu) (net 17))
 (segment (start 163.83 104.775) (end 163.83 102.87) (width 2) (layer F.Cu) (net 17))
 (segment (start 163.83 84.455) (end 163.83 87.63) (width 2) (layer B.Cu) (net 18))
 (segment (start 163.83 87.63) (end 165.735 89.535) (width 2) (layer B.Cu) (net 18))
 (segment (start 160.02 116.84) (end 160.02 111.76) (width 2) (layer B.Cu) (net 18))
 (segment (start 165.735 106.045) (end 165.735 103.505) (width 2) (layer B.Cu) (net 18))
 (segment (start 160.02 111.76) (end 165.735 106.045) (width 2) (layer B.Cu) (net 18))
 (segment (start 165.735 89.535) (end 165.735 103.505) (width 2) (layer B.Cu) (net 18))
 (segment (start 165.735 103.505) (end 165.735 104.775) (width 2) (layer B.Cu) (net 18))
 (segment (start 153.035 106.68) (end 153.035 102.87) (width 2) (layer F.Cu) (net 19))
 (segment (start 153.67 107.315) (end 153.035 106.68) (width 2) (layer F.Cu) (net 19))
 (segment (start 154.94 116.84) (end 154.94 114.3) (width 2) (layer F.Cu) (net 19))
 (segment (start 154.94 114.3) (end 154.94 111.76) (width 2) (layer F.Cu) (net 19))
 (segment (start 154.94 108.585) (end 153.67 107.315) (width 2) (layer F.Cu) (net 19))
 (segment (start 154.94 111.76) (end 154.94 108.585) (width 2) (layer F.Cu) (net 19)))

